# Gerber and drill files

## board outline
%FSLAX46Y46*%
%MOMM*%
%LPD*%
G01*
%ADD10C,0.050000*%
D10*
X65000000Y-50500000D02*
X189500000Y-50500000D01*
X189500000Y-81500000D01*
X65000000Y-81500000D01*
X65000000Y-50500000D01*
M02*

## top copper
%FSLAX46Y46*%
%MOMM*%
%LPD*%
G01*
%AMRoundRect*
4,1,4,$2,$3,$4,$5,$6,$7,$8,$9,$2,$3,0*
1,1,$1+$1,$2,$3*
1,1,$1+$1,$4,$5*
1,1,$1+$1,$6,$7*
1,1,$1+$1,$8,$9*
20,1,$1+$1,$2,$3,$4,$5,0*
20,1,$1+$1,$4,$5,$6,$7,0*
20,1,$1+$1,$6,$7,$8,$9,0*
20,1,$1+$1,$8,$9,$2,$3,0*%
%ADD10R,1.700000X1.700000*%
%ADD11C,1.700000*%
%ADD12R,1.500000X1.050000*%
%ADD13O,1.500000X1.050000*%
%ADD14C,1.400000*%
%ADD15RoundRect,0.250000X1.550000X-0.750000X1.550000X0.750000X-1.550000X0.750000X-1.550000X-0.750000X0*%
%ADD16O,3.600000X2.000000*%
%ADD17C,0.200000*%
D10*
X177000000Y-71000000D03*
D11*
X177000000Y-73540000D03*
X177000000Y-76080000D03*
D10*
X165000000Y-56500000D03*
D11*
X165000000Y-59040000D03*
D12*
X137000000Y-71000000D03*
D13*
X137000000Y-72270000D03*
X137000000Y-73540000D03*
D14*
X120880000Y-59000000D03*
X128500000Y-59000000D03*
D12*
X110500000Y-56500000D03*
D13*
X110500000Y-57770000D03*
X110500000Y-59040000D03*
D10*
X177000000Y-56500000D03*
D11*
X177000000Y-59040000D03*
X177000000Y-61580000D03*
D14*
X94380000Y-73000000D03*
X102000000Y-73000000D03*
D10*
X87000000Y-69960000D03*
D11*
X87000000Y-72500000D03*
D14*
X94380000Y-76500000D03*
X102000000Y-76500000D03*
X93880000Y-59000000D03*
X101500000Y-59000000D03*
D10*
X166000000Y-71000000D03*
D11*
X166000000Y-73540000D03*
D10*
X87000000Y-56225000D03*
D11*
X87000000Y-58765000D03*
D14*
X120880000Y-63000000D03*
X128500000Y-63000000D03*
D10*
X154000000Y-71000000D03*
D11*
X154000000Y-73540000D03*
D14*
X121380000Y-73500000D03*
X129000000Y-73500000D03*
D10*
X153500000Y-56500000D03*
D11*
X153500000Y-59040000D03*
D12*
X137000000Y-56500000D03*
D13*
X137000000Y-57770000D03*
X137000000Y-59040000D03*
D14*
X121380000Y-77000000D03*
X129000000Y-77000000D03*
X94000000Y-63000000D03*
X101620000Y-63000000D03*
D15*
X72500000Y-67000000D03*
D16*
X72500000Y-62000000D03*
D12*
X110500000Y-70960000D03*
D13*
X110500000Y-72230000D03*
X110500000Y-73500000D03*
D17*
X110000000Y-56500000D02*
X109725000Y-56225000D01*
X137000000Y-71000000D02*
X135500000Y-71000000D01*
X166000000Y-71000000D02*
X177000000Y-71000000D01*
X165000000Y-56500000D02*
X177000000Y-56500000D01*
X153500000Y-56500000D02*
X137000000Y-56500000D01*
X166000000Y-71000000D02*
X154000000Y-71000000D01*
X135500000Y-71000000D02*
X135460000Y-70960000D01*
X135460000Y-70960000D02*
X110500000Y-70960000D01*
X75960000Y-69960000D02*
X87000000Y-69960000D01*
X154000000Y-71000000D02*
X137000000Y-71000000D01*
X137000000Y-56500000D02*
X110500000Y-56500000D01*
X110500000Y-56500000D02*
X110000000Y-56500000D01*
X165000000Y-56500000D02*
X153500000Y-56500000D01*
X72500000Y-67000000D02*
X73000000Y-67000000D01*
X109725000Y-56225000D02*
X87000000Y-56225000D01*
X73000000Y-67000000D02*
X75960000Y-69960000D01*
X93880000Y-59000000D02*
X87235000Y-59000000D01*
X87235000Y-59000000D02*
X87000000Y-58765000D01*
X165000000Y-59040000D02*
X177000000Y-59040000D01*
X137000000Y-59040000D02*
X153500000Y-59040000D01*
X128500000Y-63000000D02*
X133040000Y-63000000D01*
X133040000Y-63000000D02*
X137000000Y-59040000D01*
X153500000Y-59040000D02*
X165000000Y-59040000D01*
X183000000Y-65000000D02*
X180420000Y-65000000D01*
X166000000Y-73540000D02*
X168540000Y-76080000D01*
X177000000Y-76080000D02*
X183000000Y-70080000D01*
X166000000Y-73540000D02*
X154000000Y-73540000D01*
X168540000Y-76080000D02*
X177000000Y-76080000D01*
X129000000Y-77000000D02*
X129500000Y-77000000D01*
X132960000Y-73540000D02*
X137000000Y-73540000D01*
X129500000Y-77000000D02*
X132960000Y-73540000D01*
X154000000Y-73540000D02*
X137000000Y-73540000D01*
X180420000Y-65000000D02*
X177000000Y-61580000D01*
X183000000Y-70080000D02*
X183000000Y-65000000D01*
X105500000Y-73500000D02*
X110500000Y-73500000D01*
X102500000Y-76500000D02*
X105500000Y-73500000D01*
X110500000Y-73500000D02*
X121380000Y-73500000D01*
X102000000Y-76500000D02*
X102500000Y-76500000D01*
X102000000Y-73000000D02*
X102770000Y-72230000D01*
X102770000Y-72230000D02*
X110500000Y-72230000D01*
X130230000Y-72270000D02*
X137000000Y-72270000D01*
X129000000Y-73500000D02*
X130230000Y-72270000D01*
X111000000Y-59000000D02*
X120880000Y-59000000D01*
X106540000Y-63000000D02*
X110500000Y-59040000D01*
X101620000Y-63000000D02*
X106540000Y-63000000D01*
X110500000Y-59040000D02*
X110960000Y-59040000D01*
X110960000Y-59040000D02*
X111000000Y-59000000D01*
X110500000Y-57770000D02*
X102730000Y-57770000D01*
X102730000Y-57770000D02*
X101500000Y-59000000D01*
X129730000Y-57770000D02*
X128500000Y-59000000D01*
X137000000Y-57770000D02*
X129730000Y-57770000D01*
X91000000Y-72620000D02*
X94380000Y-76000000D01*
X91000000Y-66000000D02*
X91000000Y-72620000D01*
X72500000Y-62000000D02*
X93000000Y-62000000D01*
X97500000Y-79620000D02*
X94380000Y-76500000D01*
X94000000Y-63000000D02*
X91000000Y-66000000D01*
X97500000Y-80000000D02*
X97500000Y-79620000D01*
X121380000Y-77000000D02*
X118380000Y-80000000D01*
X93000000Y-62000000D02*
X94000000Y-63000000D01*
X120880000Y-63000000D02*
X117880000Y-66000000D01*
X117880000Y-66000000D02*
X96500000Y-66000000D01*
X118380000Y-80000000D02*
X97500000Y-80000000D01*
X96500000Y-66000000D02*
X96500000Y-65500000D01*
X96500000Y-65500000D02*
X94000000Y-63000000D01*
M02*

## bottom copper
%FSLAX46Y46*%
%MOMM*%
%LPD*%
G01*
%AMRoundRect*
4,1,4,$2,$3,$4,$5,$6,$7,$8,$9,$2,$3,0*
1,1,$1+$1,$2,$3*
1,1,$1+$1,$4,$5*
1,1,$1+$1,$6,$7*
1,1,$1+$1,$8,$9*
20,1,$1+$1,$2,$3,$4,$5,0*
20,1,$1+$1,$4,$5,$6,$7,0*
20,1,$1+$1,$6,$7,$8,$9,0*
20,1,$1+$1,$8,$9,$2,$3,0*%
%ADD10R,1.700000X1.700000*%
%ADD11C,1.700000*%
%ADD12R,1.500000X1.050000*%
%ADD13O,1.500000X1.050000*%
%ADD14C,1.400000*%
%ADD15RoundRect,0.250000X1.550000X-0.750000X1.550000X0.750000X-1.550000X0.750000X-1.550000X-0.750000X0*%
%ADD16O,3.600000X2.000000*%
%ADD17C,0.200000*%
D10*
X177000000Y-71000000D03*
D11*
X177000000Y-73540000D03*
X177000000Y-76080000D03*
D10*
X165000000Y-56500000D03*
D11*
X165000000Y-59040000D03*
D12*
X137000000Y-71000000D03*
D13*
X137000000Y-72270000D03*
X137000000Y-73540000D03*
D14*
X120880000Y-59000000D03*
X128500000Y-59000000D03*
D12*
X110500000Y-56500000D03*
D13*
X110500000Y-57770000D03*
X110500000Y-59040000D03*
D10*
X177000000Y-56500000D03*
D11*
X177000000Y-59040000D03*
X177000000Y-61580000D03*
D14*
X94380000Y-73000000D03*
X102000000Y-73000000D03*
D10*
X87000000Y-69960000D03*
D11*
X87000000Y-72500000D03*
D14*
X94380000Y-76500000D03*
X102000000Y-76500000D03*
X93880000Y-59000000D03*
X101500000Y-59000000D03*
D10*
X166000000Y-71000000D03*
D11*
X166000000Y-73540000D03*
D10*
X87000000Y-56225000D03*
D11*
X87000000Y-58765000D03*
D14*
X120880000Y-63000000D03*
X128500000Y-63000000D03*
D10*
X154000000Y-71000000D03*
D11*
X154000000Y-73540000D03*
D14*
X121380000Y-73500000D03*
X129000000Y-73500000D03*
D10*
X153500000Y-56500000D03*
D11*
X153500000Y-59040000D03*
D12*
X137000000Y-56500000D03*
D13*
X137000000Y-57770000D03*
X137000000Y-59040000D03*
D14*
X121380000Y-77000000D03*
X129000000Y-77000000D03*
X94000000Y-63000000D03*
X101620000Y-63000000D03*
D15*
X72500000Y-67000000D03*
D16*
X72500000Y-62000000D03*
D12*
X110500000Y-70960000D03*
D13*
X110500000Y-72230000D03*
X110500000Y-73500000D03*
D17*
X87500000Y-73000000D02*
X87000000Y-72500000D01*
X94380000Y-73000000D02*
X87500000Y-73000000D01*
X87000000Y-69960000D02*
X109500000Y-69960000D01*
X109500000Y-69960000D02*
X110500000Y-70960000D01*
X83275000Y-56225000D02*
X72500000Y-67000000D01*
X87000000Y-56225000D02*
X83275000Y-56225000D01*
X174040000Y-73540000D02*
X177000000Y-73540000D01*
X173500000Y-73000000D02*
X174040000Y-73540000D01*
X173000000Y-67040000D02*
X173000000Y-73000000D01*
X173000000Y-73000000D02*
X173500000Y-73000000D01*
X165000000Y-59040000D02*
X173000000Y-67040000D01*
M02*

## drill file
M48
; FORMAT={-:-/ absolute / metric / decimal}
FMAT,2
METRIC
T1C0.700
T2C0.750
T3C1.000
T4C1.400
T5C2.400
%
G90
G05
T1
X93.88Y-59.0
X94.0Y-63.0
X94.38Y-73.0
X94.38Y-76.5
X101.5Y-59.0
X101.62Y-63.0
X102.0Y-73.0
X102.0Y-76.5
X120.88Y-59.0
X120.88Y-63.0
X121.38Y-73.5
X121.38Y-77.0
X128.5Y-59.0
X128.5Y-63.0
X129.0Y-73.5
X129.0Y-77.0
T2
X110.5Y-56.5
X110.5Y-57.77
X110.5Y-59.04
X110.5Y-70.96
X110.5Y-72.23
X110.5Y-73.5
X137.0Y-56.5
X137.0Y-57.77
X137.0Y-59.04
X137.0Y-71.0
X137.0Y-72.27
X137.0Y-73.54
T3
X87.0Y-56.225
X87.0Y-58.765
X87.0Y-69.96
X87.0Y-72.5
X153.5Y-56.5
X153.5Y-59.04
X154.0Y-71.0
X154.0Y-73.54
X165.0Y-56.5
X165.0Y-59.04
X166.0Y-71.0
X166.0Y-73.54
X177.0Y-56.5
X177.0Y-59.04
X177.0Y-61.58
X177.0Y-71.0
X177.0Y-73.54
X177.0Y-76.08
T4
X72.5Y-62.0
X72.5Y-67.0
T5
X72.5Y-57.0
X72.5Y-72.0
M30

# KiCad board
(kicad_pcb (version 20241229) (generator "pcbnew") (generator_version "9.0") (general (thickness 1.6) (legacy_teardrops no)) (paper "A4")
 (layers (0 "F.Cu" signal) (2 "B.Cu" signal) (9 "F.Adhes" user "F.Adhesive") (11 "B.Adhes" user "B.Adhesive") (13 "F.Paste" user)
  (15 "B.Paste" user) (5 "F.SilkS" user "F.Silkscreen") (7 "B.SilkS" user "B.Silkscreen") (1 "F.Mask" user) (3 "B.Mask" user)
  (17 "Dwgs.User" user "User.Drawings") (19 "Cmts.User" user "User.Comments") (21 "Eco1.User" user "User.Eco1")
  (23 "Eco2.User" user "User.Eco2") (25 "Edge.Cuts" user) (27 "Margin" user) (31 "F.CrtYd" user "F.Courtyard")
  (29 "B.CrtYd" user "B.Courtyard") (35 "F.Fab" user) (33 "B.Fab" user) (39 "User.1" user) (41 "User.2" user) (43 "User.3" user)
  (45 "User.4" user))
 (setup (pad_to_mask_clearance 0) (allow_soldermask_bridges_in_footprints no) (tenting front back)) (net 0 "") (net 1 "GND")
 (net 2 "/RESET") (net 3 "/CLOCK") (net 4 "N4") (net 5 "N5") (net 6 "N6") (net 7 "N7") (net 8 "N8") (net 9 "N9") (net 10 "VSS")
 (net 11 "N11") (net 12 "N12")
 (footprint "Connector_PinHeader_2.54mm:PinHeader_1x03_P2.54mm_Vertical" (layer "F.Cu") (at 177 71)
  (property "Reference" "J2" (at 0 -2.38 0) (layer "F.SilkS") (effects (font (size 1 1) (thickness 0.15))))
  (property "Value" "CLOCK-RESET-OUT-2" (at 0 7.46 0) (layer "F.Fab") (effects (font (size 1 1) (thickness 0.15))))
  (pad "1" thru_hole rect (at 0 0) (size 1.7 1.7) (drill 1) (layers "*.Cu" "*.Mask") (remove_unused_layers no) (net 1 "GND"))
  (pad "2" thru_hole circle (at 0 2.54) (size 1.7 1.7) (drill 1) (layers "*.Cu" "*.Mask") (remove_unused_layers no) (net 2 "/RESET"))
  (pad "3" thru_hole circle (at 0 5.08) (size 1.7 1.7) (drill 1) (layers "*.Cu" "*.Mask") (remove_unused_layers no) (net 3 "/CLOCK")))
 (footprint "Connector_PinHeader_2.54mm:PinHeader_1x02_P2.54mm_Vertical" (layer "F.Cu") (at 165 56.5)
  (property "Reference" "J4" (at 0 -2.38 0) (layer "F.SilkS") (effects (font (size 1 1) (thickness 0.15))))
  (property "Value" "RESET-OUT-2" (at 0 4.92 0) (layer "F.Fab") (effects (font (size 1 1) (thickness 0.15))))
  (pad "1" thru_hole rect (at 0 0) (size 1.7 1.7) (drill 1) (layers "*.Cu" "*.Mask") (remove_unused_layers no) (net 1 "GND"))
  (pad "2" thru_hole circle (at 0 2.54) (size 1.7 1.7) (drill 1) (layers "*.Cu" "*.Mask") (remove_unused_layers no) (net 2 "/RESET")))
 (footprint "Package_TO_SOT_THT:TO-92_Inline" (layer "F.Cu") (at 137 71 -90)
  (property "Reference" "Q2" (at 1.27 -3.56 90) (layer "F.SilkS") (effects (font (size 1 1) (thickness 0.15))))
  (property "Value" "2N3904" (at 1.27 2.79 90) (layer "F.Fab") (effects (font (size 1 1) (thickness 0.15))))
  (pad "1" thru_hole rect (at 0 0 270) (size 1.05 1.5) (drill 0.75) (layers "*.Cu" "*.Mask") (remove_unused_layers no) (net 1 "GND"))
  (pad "2" thru_hole oval (at 1.27 0 270) (size 1.05 1.5) (drill 0.75) (layers "*.Cu" "*.Mask") (remove_unused_layers no) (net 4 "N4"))
  (pad "3" thru_hole oval (at 2.54 0 270) (size 1.05 1.5) (drill 0.75) (layers "*.Cu" "*.Mask") (remove_unused_layers no) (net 3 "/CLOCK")))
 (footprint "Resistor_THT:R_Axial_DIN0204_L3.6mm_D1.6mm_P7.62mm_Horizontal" (layer "F.Cu") (at 120.88 59)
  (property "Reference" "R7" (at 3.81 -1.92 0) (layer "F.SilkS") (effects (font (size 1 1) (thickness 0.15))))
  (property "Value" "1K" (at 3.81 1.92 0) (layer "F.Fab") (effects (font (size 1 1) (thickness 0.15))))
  (pad "1" thru_hole circle (at 0 0) (size 1.4 1.4) (drill 0.7) (layers "*.Cu" "*.Mask") (remove_unused_layers no) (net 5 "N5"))
  (pad "2" thru_hole circle (at 7.62 0) (size 1.4 1.4) (drill 0.7) (layers "*.Cu" "*.Mask") (remove_unused_layers no) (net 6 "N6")))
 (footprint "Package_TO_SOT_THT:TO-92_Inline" (layer "F.Cu") (at 110.5 56.5 -90)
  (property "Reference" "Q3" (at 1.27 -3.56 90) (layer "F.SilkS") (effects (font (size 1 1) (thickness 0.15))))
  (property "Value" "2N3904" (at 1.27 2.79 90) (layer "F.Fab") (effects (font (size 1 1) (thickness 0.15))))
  (pad "1" thru_hole rect (at 0 0 270) (size 1.05 1.5) (drill 0.75) (layers "*.Cu" "*.Mask") (remove_unused_layers no) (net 1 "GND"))
  (pad "2" thru_hole oval (at 1.27 0 270) (size 1.05 1.5) (drill 0.75) (layers "*.Cu" "*.Mask") (remove_unused_layers no) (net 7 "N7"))
  (pad "3" thru_hole oval (at 2.54 0 270) (size 1.05 1.5) (drill 0.75) (layers "*.Cu" "*.Mask") (remove_unused_layers no) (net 5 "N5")))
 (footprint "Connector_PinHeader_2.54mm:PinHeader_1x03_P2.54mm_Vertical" (layer "F.Cu") (at 177 56.5)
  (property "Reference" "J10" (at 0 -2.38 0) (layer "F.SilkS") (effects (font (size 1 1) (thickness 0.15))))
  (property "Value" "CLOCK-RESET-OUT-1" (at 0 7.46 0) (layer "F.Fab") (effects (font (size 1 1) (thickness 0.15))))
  (pad "1" thru_hole rect (at 0 0) (size 1.7 1.7) (drill 1) (layers "*.Cu" "*.Mask") (remove_unused_layers no) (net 1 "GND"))
  (pad "2" thru_hole circle (at 0 2.54) (size 1.7 1.7) (drill 1) (layers "*.Cu" "*.Mask") (remove_unused_layers no) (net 2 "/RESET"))
  (pad "3" thru_hole circle (at 0 5.08) (size 1.7 1.7) (drill 1) (layers "*.Cu" "*.Mask") (remove_unused_layers no) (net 3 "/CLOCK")))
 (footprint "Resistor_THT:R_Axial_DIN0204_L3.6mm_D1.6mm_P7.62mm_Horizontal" (layer "F.Cu") (at 94.38 73)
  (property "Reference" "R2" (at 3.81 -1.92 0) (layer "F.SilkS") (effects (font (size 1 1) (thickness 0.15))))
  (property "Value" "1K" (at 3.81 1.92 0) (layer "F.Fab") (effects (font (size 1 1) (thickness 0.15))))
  (pad "1" thru_hole circle (at 0 0) (size 1.4 1.4) (drill 0.7) (layers "*.Cu" "*.Mask") (remove_unused_layers no) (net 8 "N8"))
  (pad "2" thru_hole circle (at 7.62 0) (size 1.4 1.4) (drill 0.7) (layers "*.Cu" "*.Mask") (remove_unused_layers no) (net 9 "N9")))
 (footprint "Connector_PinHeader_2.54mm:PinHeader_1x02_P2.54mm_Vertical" (layer "F.Cu") (at 87 69.96)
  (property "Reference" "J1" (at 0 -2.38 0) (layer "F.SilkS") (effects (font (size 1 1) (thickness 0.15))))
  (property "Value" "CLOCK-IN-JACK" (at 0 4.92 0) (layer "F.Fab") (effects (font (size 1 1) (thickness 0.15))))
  (pad "1" thru_hole rect (at 0 0) (size 1.7 1.7) (drill 1) (layers "*.Cu" "*.Mask") (remove_unused_layers no) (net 1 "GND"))
  (pad "2" thru_hole circle (at 0 2.54) (size 1.7 1.7) (drill 1) (layers "*.Cu" "*.Mask") (remove_unused_layers no) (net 8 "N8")))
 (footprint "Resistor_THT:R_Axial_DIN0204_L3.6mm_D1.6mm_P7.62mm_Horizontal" (layer "F.Cu") (at 94.38 76.5)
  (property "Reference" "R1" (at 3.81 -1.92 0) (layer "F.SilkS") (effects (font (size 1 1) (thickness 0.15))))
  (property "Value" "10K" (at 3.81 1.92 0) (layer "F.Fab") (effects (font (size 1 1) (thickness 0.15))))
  (pad "1" thru_hole circle (at 0 0) (size 1.4 1.4) (drill 0.7) (layers "*.Cu" "*.Mask") (remove_unused_layers no) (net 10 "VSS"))
  (pad "2" thru_hole circle (at 7.62 0) (size 1.4 1.4) (drill 0.7) (layers "*.Cu" "*.Mask") (remove_unused_layers no) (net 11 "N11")))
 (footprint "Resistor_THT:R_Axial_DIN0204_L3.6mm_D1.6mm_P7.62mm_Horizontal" (layer "F.Cu") (at 93.88 59)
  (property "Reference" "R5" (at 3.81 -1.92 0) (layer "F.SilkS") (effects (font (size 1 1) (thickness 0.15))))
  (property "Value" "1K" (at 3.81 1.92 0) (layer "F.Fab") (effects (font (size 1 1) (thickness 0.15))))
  (pad "1" thru_hole circle (at 0 0) (size 1.4 1.4) (drill 0.7) (layers "*.Cu" "*.Mask") (remove_unused_layers no) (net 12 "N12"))
  (pad "2" thru_hole circle (at 7.62 0) (size 1.4 1.4) (drill 0.7) (layers "*.Cu" "*.Mask") (remove_unused_layers no) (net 7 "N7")))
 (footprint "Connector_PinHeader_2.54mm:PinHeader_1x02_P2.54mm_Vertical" (layer "F.Cu") (at 166 71)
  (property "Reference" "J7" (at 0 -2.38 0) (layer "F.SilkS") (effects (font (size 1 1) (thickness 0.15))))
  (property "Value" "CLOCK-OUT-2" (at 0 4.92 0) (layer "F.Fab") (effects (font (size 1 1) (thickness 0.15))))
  (pad "1" thru_hole rect (at 0 0) (size 1.7 1.7) (drill 1) (layers "*.Cu" "*.Mask") (remove_unused_layers no) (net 1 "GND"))
  (pad "2" thru_hole circle (at 0 2.54) (size 1.7 1.7) (drill 1) (layers "*.Cu" "*.Mask") (remove_unused_layers no) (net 3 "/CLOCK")))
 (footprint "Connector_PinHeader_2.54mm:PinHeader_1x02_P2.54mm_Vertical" (layer "F.Cu") (at 87 56.225)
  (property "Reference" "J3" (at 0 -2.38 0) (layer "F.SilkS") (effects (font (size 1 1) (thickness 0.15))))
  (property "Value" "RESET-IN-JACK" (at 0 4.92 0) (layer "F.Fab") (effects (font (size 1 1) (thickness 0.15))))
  (pad "1" thru_hole rect (at 0 0) (size 1.7 1.7) (drill 1) (layers "*.Cu" "*.Mask") (remove_unused_layers no) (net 1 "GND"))
  (pad "2" thru_hole circle (at 0 2.54) (size 1.7 1.7) (drill 1) (layers "*.Cu" "*.Mask") (remove_unused_layers no) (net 12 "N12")))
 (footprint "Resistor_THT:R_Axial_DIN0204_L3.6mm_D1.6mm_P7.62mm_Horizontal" (layer "F.Cu") (at 120.88 63)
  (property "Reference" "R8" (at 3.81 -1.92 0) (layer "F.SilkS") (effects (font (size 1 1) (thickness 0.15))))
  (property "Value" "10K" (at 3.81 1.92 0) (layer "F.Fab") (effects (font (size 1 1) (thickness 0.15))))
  (pad "1" thru_hole circle (at 0 0) (size 1.4 1.4) (drill 0.7) (layers "*.Cu" "*.Mask") (remove_unused_layers no) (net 10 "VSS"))
  (pad "2" thru_hole circle (at 7.62 0) (size 1.4 1.4) (drill 0.7) (layers "*.Cu" "*.Mask") (remove_unused_layers no) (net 2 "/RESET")))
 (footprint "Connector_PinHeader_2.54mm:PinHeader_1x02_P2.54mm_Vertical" (layer "F.Cu") (at 154 71)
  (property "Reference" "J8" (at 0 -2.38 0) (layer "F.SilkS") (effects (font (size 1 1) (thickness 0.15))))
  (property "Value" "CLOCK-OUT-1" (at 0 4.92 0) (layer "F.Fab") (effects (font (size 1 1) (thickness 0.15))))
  (pad "1" thru_hole rect (at 0 0) (size 1.7 1.7) (drill 1) (layers "*.Cu" "*.Mask") (remove_unused_layers no) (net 1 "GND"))
  (pad "2" thru_hole circle (at 0 2.54) (size 1.7 1.7) (drill 1) (layers "*.Cu" "*.Mask") (remove_unused_layers no) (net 3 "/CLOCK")))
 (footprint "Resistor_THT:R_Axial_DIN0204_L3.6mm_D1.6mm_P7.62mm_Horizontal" (layer "F.Cu") (at 121.38 73.5)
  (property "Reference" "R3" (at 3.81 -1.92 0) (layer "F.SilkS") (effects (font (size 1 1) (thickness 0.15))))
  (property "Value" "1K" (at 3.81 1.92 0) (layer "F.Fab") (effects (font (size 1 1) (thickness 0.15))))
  (pad "1" thru_hole circle (at 0 0) (size 1.4 1.4) (drill 0.7) (layers "*.Cu" "*.Mask") (remove_unused_layers no) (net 11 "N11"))
  (pad "2" thru_hole circle (at 7.62 0) (size 1.4 1.4) (drill 0.7) (layers "*.Cu" "*.Mask") (remove_unused_layers no) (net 4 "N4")))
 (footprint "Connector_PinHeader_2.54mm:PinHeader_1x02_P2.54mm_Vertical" (layer "F.Cu") (at 153.5 56.5)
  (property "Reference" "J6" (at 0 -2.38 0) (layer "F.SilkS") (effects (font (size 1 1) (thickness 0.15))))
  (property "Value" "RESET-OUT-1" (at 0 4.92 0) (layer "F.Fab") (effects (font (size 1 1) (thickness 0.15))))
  (pad "1" thru_hole rect (at 0 0) (size 1.7 1.7) (drill 1) (layers "*.Cu" "*.Mask") (remove_unused_layers no) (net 1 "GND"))
  (pad "2" thru_hole circle (at 0 2.54) (size 1.7 1.7) (drill 1) (layers "*.Cu" "*.Mask") (remove_unused_layers no) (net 2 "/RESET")))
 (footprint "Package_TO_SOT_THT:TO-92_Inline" (layer "F.Cu") (at 137 56.5 -90)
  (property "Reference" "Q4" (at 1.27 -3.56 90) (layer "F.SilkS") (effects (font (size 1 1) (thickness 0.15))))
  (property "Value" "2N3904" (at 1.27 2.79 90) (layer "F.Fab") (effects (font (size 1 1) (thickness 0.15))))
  (pad "1" thru_hole rect (at 0 0 270) (size 1.05 1.5) (drill 0.75) (layers "*.Cu" "*.Mask") (remove_unused_layers no) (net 1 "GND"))
  (pad "2" thru_hole oval (at 1.27 0 270) (size 1.05 1.5) (drill 0.75) (layers "*.Cu" "*.Mask") (remove_unused_layers no) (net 6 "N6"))
  (pad "3" thru_hole oval (at 2.54 0 270) (size 1.05 1.5) (drill 0.75) (layers "*.Cu" "*.Mask") (remove_unused_layers no) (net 2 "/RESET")))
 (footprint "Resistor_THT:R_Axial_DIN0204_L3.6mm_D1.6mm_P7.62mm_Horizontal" (layer "F.Cu") (at 121.38 77)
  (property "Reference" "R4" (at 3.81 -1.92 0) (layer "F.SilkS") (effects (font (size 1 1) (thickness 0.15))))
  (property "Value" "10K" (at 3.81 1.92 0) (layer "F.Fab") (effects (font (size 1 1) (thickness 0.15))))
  (pad "1" thru_hole circle (at 0 0) (size 1.4 1.4) (drill 0.7) (layers "*.Cu" "*.Mask") (remove_unused_layers no) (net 10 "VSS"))
  (pad "2" thru_hole circle (at 7.62 0) (size 1.4 1.4) (drill 0.7) (layers "*.Cu" "*.Mask") (remove_unused_layers no) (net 3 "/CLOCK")))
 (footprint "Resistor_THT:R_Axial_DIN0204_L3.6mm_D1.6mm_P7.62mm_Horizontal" (layer "F.Cu") (at 94 63)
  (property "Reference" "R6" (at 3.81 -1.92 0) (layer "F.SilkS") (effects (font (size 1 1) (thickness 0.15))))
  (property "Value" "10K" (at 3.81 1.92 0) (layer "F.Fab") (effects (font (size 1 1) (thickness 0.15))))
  (pad "1" thru_hole circle (at 0 0) (size 1.4 1.4) (drill 0.7) (layers "*.Cu" "*.Mask") (remove_unused_layers no) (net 10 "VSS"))
  (pad "2" thru_hole circle (at 7.62 0) (size 1.4 1.4) (drill 0.7) (layers "*.Cu" "*.Mask") (remove_unused_layers no) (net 5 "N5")))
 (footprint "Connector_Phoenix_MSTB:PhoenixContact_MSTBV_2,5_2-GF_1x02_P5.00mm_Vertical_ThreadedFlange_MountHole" (layer "F.Cu")
  (at 72.5 67 90)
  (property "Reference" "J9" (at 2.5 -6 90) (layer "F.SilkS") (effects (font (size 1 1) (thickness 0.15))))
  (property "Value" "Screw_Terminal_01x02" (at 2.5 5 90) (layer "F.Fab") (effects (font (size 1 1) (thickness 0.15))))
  (pad "" np_thru_hole circle (at -5 0 90) (size 2.4 2.4) (drill 2.4) (layers "*.Cu" "*.Mask"))
  (pad "" np_thru_hole circle (at 10 0 90) (size 2.4 2.4) (drill 2.4) (layers "*.Cu" "*.Mask"))
  (pad "1" thru_hole roundrect (at 0 0 90) (size 2 3.6) (drill 1.4) (layers "*.Cu" "*.Mask") (remove_unused_layers no)
   (roundrect_rratio 0.125) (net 1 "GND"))
  (pad "2" thru_hole oval (at 5 0 90) (size 2 3.6) (drill 1.4) (layers "*.Cu" "*.Mask") (remove_unused_layers no) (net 10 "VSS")))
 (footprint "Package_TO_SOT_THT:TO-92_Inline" (layer "F.Cu") (at 110.5 70.96 -90)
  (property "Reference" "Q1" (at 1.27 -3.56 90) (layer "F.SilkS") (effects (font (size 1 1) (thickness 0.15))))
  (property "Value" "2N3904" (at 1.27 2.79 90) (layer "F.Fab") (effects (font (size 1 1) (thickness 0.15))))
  (pad "1" thru_hole rect (at 0 0 270) (size 1.05 1.5) (drill 0.75) (layers "*.Cu" "*.Mask") (remove_unused_layers no) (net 1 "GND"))
  (pad "2" thru_hole oval (at 1.27 0 270) (size 1.05 1.5) (drill 0.75) (layers "*.Cu" "*.Mask") (remove_unused_layers no) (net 9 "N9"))
  (pad "3" thru_hole oval (at 2.54 0 270) (size 1.05 1.5) (drill 0.75) (layers "*.Cu" "*.Mask") (remove_unused_layers no) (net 11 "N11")))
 (gr_rect (start 65 50.5) (end 189.5 81.5) (stroke (width 0.05) (type default)) (fill no) (layer "Edge.Cuts"))
 (segment (start 87.5 73) (end 87 72.5) (width 0.2) (layer "B.Cu") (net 8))
 (segment (start 94.38 73) (end 87.5 73) (width 0.2) (layer "B.Cu") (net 8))
 (segment (start 110 56.5) (end 109.725 56.225) (width 0.2) (layer "F.Cu") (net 1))
 (segment (start 137 71) (end 135.5 71) (width 0.2) (layer "F.Cu") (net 1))
 (segment (start 166 71) (end 177 71) (width 0.2) (layer "F.Cu") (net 1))
 (segment (start 165 56.5) (end 177 56.5) (width 0.2) (layer "F.Cu") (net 1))
 (segment (start 153.5 56.5) (end 137 56.5) (width 0.2) (layer "F.Cu") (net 1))
 (segment (start 166 71) (end 154 71) (width 0.2) (layer "F.Cu") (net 1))
 (segment (start 135.5 71) (end 135.46 70.96) (width 0.2) (layer "F.Cu") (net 1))
 (segment (start 135.46 70.96) (end 110.5 70.96) (width 0.2) (layer "F.Cu") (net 1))
 (segment (start 75.96 69.96) (end 87 69.96) (width 0.2) (layer "F.Cu") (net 1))
 (segment (start 154 71) (end 137 71) (width 0.2) (layer "F.Cu") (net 1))
 (segment (start 137 56.5) (end 110.5 56.5) (width 0.2) (layer "F.Cu") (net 1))
 (segment (start 110.5 56.5) (end 110 56.5) (width 0.2) (layer "F.Cu") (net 1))
 (segment (start 165 56.5) (end 153.5 56.5) (width 0.2) (layer "F.Cu") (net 1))
 (segment (start 72.5 67) (end 73 67) (width 0.2) (layer "F.Cu") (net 1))
 (segment (start 109.725 56.225) (end 87 56.225) (width 0.2) (layer "F.Cu") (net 1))
 (segment (start 73 67) (end 75.96 69.96) (width 0.2) (layer "F.Cu") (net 1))
 (segment (start 87 69.96) (end 109.5 69.96) (width 0.2) (layer "B.Cu") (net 1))
 (segment (start 109.5 69.96) (end 110.5 70.96) (width 0.2) (layer "B.Cu") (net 1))
 (segment (start 83.275 56.225) (end 72.5 67) (width 0.2) (layer "B.Cu") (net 1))
 (segment (start 87 56.225) (end 83.275 56.225) (width 0.2) (layer "B.Cu") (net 1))
 (segment (start 93.88 59) (end 87.235 59) (width 0.2) (layer "F.Cu") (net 12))
 (segment (start 87.235 59) (end 87 58.765) (width 0.2) (layer "F.Cu") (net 12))
 (segment (start 165 59.04) (end 177 59.04) (width 0.2) (layer "F.Cu") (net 2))
 (segment (start 137 59.04) (end 153.5 59.04) (width 0.2) (layer "F.Cu") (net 2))
 (segment (start 128.5 63) (end 133.04 63) (width 0.2) (layer "F.Cu") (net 2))
 (segment (start 133.04 63) (end 137 59.04) (width 0.2) (layer "F.Cu") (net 2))
 (segment (start 153.5 59.04) (end 165 59.04) (width 0.2) (layer "F.Cu") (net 2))
 (segment (start 174.04 73.54) (end 177 73.54) (width 0.2) (layer "B.Cu") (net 2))
 (segment (start 173.5 73) (end 174.04 73.54) (width 0.2) (layer "B.Cu") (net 2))
 (segment (start 173 67.04) (end 173 73) (width 0.2) (layer "B.Cu") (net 2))
 (segment (start 173 73) (end 173.5 73) (width 0.2) (layer "B.Cu") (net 2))
 (segment (start 165 59.04) (end 173 67.04) (width 0.2) (layer "B.Cu") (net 2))
 (segment (start 183 65) (end 180.42 65) (width 0.2) (layer "F.Cu") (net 3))
 (segment (start 166 73.54) (end 168.54 76.08) (width 0.2) (layer "F.Cu") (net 3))
 (segment (start 177 76.08) (end 183 70.08) (width 0.2) (layer "F.Cu") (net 3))
 (segment (start 166 73.54) (end 154 73.54) (width 0.2) (layer "F.Cu") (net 3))
 (segment (start 168.54 76.08) (end 177 76.08) (width 0.2) (layer "F.Cu") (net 3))
 (segment (start 129 77) (end 129.5 77) (width 0.2) (layer "F.Cu") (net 3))
 (segment (start 132.96 73.54) (end 137 73.54) (width 0.2) (layer "F.Cu") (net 3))
 (segment (start 129.5 77) (end 132.96 73.54) (width 0.2) (layer "F.Cu") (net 3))
 (segment (start 154 73.54) (end 137 73.54) (width 0.2) (layer "F.Cu") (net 3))
 (segment (start 180.42 65) (end 177 61.58) (width 0.2) (layer "F.Cu") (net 3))
 (segment (start 183 70.08) (end 183 65) (width 0.2) (layer "F.Cu") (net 3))
 (segment (start 105.5 73.5) (end 110.5 73.5) (width 0.2) (layer "F.Cu") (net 11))
 (segment (start 102.5 76.5) (end 105.5 73.5) (width 0.2) (layer "F.Cu") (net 11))
 (segment (start 110.5 73.5) (end 121.38 73.5) (width 0.2) (layer "F.Cu") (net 11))
 (segment (start 102 76.5) (end 102.5 76.5) (width 0.2) (layer "F.Cu") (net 11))
 (segment (start 102 73) (end 102.77 72.23) (width 0.2) (layer "F.Cu") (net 9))
 (segment (start 102.77 72.23) (end 110.5 72.23) (width 0.2) (layer "F.Cu") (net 9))
 (segment (start 130.23 72.27) (end 137 72.27) (width 0.2) (layer "F.Cu") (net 4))
 (segment (start 129 73.5) (end 130.23 72.27) (width 0.2) (layer "F.Cu") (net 4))
 (segment (start 111 59) (end 120.88 59) (width 0.2) (layer "F.Cu") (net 5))
 (segment (start 106.54 63) (end 110.5 59.04) (width 0.2) (layer "F.Cu") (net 5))
 (segment (start 101.62 63) (end 106.54 63) (width 0.2) (layer "F.Cu") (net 5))
 (segment (start 110.5 59.04) (end 110.96 59.04) (width 0.2) (layer "F.Cu") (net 5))
 (segment (start 110.96 59.04) (end 111 59) (width 0.2) (layer "F.Cu") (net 5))
 (segment (start 110.5 57.77) (end 102.73 57.77) (width 0.2) (layer "F.Cu") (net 7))
 (segment (start 102.73 57.77) (end 101.5 59) (width 0.2) (layer "F.Cu") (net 7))
 (segment (start 129.73 57.77) (end 128.5 59) (width 0.2) (layer "F.Cu") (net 6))
 (segment (start 137 57.77) (end 129.73 57.77) (width 0.2) (layer "F.Cu") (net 6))
 (segment (start 91 72.62) (end 94.38 76) (width 0.2) (layer "F.Cu") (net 10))
 (segment (start 91 66) (end 91 72.62) (width 0.2) (layer "F.Cu") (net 10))
 (segment (start 72.5 62) (end 93 62) (width 0.2) (layer "F.Cu") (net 10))
 (segment (start 97.5 79.62) (end 94.38 76.5) (width 0.2) (layer "F.Cu") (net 10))
 (segment (start 94 63) (end 91 66) (width 0.2) (layer "F.Cu") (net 10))
 (segment (start 97.5 80) (end 97.5 79.62) (width 0.2) (layer "F.Cu") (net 10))
 (segment (start 121.38 77) (end 118.38 80) (width 0.2) (layer "F.Cu") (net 10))
 (segment (start 93 62) (end 94 63) (width 0.2) (layer "F.Cu") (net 10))
 (segment (start 120.88 63) (end 117.88 66) (width 0.2) (layer "F.Cu") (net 10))
 (segment (start 117.88 66) (end 96.5 66) (width 0.2) (layer "F.Cu") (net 10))
 (segment (start 118.38 80) (end 97.5 80) (width 0.2) (layer "F.Cu") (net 10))
 (segment (start 96.5 66) (end 96.5 65.5) (width 0.2) (layer "F.Cu") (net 10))
 (segment (start 96.5 65.5) (end 94 63) (width 0.2) (layer "F.Cu") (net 10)))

